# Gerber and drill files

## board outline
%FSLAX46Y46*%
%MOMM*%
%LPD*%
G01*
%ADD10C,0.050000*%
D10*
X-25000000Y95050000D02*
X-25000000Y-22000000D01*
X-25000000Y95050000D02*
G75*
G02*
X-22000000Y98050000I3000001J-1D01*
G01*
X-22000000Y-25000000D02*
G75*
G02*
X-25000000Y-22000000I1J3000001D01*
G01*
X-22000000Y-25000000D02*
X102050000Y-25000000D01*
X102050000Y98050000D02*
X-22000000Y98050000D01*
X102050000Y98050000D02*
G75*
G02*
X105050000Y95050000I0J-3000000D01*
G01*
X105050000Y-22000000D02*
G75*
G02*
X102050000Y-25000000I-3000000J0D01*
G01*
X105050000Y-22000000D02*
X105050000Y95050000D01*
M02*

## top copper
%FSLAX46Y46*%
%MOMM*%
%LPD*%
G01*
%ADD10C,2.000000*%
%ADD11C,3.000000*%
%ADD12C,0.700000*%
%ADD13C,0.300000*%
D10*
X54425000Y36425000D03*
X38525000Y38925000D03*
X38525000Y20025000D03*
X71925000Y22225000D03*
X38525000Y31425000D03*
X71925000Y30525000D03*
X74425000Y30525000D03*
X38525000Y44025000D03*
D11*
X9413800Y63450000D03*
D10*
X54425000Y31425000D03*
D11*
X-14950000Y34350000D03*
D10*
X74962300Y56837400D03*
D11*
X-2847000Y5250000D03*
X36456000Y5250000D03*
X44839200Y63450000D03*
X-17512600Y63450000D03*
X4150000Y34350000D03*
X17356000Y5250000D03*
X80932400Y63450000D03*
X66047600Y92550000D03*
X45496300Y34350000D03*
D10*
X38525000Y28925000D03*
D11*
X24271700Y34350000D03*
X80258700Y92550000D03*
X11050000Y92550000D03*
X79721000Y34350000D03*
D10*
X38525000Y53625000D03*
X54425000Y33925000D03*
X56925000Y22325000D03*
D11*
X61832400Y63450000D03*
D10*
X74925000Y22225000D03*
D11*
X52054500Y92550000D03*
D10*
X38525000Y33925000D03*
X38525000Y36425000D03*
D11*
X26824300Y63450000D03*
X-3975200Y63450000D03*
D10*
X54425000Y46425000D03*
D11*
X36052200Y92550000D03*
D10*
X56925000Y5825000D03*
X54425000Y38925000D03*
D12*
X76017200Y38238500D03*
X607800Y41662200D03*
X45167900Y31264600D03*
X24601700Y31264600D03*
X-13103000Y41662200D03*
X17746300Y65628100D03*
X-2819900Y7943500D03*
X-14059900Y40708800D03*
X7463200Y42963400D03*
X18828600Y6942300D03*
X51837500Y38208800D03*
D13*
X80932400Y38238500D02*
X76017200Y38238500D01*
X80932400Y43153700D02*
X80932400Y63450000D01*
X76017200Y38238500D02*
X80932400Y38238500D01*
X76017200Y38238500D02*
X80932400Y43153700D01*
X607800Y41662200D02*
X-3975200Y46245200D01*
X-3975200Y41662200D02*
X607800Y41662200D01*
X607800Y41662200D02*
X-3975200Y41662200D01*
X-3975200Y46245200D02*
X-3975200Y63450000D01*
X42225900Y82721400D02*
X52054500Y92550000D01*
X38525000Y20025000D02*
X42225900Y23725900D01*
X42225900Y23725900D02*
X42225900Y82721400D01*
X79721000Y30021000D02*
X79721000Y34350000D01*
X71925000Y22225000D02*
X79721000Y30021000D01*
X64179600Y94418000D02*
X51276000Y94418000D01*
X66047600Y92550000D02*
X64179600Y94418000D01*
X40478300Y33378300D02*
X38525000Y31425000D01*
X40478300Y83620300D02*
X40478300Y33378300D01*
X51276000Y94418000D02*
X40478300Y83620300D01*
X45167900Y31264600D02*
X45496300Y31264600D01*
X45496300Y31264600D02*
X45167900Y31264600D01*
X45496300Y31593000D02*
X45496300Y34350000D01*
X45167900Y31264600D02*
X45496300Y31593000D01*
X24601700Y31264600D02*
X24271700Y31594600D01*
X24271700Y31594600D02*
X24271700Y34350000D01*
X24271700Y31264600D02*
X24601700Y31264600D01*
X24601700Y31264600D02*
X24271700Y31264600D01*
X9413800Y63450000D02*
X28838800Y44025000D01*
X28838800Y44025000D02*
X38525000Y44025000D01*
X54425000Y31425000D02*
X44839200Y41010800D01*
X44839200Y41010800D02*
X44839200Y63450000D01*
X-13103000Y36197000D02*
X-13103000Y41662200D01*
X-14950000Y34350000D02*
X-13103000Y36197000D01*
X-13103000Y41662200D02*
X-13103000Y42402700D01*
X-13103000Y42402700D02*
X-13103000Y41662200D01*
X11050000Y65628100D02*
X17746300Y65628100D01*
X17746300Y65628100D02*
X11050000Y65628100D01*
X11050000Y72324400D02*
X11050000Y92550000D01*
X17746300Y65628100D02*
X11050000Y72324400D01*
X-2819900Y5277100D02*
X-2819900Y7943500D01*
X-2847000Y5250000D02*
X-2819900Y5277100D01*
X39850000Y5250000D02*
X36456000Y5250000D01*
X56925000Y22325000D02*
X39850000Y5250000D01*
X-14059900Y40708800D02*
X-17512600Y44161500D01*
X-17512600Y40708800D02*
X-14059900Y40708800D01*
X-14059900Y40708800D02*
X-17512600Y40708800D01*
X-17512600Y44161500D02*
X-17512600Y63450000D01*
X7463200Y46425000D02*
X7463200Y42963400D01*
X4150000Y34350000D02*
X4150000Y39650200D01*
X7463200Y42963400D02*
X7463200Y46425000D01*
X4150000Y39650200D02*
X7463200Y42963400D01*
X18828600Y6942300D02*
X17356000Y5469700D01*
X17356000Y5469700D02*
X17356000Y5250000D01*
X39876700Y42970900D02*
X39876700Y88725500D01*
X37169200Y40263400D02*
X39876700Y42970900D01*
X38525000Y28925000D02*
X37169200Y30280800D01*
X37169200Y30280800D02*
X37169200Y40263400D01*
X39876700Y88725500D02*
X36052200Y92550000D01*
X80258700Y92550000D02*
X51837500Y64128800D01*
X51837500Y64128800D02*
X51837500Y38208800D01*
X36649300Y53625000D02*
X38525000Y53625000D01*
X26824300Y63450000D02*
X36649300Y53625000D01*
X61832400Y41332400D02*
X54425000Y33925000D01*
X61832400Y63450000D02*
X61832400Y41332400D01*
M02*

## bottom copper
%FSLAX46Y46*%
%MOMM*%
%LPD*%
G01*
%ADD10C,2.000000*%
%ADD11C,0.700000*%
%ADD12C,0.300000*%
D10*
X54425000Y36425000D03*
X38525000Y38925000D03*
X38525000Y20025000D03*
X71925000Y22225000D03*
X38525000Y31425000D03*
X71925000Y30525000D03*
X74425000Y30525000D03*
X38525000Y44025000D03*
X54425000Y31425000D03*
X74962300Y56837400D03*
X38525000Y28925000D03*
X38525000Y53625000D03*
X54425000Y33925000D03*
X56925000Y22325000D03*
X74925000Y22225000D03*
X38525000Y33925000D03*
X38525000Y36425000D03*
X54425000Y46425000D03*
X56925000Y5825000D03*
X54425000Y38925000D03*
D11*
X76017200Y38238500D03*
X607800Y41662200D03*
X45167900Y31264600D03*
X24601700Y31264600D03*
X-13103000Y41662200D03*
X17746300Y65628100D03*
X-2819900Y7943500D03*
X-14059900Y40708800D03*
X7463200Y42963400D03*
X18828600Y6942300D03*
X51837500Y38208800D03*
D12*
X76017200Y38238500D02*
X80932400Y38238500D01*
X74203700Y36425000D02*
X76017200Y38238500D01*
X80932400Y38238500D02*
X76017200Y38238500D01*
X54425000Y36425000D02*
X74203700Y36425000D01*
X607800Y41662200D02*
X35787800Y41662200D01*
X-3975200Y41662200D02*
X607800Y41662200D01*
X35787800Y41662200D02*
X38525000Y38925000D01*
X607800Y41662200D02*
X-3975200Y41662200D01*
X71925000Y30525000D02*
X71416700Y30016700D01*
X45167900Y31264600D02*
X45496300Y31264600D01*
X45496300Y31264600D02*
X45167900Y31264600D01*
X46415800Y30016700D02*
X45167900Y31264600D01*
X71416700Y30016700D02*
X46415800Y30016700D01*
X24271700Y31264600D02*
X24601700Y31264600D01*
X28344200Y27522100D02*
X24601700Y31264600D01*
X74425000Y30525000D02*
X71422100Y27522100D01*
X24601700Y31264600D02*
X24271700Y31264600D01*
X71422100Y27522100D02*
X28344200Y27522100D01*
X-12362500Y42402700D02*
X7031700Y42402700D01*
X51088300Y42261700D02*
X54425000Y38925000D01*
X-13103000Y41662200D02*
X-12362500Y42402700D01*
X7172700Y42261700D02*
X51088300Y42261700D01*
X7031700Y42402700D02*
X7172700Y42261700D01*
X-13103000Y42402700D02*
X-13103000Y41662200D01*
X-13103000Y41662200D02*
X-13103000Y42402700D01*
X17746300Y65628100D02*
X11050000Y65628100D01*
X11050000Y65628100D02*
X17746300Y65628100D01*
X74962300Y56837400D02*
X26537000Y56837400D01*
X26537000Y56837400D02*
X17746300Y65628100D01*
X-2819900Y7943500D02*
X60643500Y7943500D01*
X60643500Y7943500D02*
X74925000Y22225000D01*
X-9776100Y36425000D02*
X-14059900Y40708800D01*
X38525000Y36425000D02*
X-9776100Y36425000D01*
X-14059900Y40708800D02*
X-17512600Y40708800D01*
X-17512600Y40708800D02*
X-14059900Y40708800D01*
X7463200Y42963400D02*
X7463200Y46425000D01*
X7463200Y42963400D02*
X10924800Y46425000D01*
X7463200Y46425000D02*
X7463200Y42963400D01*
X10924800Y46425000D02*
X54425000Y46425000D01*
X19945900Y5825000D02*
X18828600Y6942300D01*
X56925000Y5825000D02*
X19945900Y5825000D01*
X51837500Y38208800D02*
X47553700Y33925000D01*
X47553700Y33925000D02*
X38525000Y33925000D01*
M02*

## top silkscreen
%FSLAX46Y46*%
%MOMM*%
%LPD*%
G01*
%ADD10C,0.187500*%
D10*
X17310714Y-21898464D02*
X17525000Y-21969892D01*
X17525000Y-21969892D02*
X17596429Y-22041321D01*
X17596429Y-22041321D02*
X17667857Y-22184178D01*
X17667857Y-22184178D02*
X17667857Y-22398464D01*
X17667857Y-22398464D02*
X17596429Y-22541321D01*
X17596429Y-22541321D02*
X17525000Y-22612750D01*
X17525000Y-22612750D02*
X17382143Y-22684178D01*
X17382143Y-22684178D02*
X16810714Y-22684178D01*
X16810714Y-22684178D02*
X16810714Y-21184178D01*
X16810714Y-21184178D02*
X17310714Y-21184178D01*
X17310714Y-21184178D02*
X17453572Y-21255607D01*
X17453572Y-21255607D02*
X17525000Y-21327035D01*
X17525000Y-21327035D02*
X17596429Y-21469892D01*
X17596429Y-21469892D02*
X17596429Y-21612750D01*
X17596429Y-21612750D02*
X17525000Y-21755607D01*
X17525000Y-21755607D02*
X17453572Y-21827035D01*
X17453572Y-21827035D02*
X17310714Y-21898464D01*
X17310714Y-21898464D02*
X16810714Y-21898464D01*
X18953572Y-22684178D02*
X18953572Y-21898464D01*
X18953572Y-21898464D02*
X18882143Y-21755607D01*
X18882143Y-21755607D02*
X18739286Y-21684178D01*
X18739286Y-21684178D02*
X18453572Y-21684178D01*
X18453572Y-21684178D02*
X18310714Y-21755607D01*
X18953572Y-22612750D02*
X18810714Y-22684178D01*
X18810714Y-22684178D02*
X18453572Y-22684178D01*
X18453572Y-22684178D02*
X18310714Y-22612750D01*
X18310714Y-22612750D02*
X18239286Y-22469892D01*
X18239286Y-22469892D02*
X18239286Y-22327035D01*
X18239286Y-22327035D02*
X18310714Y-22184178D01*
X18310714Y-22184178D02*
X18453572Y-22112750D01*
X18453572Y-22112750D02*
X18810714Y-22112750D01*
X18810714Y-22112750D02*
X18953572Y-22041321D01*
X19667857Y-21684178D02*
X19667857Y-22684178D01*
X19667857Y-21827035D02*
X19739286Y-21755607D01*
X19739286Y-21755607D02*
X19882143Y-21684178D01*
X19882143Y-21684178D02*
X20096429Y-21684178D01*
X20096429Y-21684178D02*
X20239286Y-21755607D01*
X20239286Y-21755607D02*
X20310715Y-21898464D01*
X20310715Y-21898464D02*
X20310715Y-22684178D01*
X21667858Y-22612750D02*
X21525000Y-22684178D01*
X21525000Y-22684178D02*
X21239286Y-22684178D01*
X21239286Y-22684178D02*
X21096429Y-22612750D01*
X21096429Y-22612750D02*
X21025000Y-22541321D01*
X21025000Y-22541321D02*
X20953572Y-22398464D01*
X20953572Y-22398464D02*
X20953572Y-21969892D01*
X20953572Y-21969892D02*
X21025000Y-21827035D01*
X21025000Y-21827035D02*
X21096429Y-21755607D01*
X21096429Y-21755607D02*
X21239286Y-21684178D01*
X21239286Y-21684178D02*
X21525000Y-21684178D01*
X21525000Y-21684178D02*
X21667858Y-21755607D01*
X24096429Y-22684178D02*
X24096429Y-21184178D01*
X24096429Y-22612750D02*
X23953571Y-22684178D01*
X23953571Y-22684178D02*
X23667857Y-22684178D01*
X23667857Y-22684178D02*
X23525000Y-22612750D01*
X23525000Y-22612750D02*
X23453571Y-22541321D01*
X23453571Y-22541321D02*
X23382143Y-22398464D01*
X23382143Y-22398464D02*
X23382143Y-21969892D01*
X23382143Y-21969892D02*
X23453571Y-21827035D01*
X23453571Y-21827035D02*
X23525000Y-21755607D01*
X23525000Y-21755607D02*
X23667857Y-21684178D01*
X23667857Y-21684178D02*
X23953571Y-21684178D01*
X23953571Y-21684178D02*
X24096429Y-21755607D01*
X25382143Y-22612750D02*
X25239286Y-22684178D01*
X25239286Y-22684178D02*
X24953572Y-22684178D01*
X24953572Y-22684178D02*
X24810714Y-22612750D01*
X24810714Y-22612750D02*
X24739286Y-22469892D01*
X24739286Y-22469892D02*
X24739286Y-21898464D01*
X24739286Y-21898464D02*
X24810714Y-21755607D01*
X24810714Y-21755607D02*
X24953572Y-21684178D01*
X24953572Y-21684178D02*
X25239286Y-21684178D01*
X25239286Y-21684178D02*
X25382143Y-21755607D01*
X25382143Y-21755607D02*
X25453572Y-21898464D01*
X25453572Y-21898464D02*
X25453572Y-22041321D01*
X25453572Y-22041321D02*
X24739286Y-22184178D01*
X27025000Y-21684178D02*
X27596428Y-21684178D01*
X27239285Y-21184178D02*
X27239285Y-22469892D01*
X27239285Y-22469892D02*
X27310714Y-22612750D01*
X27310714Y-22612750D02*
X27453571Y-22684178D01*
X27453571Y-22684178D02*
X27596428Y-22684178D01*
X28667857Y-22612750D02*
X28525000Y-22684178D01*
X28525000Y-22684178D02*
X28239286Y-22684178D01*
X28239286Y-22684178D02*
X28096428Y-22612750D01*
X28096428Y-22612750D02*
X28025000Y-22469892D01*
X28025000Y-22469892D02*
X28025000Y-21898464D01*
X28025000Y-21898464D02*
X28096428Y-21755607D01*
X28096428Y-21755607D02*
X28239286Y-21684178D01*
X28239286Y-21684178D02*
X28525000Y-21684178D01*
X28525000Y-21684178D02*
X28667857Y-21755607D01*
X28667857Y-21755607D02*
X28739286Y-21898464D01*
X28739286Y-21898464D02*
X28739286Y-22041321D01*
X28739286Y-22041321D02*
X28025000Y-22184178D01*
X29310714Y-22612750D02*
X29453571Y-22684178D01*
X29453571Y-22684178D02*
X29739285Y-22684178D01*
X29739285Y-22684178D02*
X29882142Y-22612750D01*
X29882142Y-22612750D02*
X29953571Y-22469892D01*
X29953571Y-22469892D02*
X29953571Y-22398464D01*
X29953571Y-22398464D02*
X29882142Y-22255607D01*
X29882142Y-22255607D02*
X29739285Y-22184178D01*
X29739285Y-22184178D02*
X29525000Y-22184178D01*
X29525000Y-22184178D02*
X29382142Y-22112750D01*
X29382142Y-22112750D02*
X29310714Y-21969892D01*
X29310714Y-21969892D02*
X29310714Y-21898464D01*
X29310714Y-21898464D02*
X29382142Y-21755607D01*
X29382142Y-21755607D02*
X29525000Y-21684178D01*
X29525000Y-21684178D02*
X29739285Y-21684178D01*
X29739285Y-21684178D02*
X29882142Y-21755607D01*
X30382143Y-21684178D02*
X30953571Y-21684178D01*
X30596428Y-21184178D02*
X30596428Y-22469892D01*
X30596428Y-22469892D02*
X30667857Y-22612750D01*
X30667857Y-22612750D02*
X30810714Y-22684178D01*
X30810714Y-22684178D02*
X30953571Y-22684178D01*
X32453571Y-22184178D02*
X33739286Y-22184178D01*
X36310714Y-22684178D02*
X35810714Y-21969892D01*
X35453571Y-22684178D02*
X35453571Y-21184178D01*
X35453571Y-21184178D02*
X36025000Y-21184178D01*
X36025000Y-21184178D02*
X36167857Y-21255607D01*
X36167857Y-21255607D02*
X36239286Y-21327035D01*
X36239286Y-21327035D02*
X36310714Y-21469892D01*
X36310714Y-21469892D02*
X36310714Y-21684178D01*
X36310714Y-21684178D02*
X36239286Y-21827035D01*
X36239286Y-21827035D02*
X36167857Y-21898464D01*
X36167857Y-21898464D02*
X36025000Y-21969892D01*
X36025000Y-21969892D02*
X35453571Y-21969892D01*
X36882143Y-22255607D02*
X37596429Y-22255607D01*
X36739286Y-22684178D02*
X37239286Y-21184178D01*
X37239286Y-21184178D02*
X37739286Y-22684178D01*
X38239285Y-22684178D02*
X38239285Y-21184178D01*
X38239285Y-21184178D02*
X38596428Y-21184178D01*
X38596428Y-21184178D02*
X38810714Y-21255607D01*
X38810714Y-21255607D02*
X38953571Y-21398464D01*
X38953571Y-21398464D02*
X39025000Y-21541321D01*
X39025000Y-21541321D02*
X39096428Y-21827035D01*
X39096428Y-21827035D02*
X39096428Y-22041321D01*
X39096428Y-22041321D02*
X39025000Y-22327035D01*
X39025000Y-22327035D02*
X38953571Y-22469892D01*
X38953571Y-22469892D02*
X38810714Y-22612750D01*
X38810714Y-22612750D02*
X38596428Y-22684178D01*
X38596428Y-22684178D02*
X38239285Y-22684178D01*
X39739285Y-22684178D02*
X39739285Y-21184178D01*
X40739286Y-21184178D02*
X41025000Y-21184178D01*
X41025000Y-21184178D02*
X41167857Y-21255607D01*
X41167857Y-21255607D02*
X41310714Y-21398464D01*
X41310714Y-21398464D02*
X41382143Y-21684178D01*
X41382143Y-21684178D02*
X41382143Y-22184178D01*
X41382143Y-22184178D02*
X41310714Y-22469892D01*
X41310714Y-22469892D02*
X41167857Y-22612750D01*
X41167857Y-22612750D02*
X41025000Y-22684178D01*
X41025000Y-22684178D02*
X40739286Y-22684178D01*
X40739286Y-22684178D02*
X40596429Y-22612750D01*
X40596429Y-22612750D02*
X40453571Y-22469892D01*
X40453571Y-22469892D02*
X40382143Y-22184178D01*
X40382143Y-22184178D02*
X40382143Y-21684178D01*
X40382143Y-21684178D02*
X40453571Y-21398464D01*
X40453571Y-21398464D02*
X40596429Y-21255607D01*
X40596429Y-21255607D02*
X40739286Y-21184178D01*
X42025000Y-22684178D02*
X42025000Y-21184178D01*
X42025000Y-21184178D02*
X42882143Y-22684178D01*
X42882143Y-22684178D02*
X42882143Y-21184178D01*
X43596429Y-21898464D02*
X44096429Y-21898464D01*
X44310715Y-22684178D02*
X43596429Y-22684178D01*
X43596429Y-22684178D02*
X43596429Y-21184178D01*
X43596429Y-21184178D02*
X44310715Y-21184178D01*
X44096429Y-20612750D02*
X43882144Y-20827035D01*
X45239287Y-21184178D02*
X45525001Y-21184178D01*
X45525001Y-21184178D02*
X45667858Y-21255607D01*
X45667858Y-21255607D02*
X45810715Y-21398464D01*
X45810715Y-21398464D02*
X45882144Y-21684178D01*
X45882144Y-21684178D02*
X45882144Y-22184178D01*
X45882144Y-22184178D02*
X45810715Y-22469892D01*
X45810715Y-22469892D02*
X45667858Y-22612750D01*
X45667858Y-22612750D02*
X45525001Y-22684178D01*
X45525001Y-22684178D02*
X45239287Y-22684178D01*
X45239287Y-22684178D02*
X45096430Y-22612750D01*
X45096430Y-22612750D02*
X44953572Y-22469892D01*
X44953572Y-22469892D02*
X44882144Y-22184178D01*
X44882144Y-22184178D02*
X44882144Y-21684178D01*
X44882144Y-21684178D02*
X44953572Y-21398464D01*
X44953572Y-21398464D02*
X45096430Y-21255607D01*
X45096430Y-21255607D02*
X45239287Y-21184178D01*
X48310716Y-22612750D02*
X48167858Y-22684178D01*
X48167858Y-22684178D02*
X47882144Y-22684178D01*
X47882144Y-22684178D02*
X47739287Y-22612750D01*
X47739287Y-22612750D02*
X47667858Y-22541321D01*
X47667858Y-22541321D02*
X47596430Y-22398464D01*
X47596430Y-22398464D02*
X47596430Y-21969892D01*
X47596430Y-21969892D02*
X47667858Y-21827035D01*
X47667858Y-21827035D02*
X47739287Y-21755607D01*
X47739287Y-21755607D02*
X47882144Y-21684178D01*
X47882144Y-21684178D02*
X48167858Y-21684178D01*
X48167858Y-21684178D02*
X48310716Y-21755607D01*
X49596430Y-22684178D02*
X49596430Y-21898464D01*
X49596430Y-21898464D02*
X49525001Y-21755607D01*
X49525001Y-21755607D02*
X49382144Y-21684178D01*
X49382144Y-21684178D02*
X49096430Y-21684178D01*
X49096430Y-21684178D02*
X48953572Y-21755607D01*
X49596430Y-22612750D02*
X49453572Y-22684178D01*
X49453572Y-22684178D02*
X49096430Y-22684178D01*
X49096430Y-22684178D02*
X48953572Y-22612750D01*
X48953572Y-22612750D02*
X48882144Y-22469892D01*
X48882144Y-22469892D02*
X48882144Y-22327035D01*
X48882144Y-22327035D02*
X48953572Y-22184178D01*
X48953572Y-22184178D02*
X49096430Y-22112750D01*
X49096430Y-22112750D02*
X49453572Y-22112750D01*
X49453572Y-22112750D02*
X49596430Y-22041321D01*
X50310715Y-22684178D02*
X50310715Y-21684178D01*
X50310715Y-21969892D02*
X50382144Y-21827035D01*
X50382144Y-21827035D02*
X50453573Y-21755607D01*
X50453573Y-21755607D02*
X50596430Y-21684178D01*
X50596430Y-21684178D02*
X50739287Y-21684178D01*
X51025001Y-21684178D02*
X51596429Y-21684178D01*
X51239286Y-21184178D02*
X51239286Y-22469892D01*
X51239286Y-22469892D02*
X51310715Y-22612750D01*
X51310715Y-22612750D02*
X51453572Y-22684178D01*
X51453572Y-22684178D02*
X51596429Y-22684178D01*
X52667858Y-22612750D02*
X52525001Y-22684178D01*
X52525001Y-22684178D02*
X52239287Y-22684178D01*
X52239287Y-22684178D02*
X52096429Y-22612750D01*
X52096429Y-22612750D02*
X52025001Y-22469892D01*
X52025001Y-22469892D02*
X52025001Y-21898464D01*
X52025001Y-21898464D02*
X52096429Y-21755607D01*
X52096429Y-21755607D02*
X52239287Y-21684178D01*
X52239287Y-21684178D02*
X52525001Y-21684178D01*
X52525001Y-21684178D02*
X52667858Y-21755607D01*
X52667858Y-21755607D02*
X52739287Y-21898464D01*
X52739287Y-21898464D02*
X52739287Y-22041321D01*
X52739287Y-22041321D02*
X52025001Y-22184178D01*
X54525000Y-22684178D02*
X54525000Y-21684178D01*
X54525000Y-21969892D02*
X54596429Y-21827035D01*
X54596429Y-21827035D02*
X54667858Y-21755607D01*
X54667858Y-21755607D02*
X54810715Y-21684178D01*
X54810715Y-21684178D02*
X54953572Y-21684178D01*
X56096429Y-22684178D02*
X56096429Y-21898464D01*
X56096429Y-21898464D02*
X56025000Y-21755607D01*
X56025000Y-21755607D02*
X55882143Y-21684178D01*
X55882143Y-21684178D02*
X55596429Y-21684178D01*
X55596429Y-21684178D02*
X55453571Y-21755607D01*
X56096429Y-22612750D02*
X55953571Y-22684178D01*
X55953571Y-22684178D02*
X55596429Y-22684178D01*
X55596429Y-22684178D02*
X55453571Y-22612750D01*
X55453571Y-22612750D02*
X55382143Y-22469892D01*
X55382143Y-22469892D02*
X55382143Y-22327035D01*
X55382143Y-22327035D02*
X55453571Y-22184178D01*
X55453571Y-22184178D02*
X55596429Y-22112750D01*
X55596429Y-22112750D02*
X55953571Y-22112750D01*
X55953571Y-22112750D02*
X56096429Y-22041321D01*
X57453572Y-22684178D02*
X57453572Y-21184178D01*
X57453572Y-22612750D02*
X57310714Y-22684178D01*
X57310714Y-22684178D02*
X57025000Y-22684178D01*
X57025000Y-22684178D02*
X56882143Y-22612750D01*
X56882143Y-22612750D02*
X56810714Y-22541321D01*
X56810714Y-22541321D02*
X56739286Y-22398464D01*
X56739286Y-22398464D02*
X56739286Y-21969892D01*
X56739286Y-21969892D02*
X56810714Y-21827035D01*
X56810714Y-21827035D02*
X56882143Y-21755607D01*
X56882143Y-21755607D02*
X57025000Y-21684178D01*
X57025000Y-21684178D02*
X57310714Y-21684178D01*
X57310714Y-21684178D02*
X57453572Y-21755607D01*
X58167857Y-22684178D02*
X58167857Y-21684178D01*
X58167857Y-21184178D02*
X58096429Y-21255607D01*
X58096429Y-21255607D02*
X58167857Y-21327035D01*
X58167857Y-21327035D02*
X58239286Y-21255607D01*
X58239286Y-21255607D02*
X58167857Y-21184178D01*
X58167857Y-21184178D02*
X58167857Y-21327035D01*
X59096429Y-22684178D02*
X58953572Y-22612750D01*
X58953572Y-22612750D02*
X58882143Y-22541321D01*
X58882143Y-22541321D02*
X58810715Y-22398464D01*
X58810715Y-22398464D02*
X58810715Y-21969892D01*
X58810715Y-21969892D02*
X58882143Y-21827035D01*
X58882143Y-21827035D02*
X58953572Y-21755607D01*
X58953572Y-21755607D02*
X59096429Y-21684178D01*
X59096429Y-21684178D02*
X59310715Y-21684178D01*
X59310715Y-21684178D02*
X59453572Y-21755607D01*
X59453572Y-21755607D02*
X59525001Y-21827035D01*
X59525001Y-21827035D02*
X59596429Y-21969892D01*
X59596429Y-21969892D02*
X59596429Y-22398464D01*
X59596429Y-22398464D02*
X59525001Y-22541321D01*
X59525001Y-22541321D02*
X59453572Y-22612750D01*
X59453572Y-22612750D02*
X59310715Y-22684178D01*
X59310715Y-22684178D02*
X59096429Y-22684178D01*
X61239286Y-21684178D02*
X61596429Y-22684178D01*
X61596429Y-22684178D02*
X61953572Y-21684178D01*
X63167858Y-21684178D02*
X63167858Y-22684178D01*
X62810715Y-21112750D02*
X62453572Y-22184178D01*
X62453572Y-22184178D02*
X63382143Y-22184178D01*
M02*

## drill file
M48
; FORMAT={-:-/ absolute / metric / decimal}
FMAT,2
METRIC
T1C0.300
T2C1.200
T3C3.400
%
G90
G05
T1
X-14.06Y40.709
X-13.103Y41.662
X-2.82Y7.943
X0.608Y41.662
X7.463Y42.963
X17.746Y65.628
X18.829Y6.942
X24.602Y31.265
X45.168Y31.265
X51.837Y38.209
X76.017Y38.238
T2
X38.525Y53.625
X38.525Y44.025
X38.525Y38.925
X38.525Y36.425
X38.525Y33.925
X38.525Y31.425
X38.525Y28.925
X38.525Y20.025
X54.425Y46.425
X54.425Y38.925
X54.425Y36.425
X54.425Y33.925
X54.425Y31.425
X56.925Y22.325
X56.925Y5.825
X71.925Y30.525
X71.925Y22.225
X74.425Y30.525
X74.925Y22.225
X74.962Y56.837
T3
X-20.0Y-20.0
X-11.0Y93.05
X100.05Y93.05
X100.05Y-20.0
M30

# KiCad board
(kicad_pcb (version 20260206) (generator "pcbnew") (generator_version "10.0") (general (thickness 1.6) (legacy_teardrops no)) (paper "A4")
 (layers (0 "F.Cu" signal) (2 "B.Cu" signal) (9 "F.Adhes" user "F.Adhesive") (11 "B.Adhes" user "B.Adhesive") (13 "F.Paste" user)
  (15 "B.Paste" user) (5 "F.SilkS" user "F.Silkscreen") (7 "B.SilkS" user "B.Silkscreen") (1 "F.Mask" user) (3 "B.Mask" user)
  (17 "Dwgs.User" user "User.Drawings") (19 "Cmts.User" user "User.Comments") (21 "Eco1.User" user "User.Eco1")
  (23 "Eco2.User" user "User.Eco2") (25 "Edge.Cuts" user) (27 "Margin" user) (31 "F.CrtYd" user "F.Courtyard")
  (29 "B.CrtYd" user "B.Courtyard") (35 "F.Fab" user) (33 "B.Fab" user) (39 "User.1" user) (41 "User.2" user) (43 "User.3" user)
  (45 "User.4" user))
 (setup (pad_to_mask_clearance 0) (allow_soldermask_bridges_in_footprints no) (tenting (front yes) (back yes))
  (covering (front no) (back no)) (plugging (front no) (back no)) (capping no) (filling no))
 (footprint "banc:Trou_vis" (layer "F.Cu") (at 100.05 -93.05)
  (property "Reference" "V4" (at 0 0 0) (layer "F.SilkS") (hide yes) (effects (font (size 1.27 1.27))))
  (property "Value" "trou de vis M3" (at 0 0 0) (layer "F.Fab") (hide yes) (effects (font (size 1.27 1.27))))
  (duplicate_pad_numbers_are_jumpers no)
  (pad "" np_thru_hole circle (at 0 0) (size 3.4 3.4) (drill 3.4) (layers "*.Cu" "*.Mask")))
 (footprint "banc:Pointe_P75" (layer "F.Cu") (at 54.425 -36.425)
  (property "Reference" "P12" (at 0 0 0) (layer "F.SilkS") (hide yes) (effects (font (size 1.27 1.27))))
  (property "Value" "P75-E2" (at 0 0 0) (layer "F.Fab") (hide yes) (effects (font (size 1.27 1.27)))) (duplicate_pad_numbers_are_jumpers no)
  (pad "1" thru_hole circle (at 0 0) (size 2 2) (drill 1.2) (layers "*.Cu" "*.Mask") (remove_unused_layers no) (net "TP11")))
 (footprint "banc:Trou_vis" (layer "F.Cu") (at 100.05 20)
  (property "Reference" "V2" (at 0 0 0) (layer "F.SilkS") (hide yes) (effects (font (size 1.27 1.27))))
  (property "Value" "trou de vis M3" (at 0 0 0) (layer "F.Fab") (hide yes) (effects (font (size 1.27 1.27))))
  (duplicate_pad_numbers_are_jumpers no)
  (pad "" np_thru_hole circle (at 0 0) (size 3.4 3.4) (drill 3.4) (layers "*.Cu" "*.Mask")))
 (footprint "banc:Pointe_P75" (layer "F.Cu") (at 38.525 -38.925)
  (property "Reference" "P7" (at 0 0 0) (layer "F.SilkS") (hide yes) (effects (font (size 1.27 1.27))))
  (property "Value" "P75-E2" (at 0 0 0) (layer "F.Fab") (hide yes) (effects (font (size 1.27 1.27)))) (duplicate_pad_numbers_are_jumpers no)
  (pad "1" thru_hole circle (at 0 0) (size 2 2) (drill 1.2) (layers "*.Cu" "*.Mask") (remove_unused_layers no) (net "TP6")))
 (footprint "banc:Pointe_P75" (layer "F.Cu") (at 38.525 -20.025)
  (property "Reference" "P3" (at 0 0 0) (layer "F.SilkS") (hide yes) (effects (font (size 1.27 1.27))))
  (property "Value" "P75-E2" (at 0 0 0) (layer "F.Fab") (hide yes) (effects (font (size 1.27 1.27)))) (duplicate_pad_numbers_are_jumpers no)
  (pad "1" thru_hole circle (at 0 0) (size 2 2) (drill 1.2) (layers "*.Cu" "*.Mask") (remove_unused_layers no) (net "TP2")))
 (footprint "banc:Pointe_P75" (layer "F.Cu") (at 71.925 -22.225)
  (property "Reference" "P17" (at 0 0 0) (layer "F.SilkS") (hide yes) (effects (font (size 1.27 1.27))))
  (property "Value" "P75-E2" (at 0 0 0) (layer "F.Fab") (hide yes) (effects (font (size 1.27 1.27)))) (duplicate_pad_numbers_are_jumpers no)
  (pad "1" thru_hole circle (at 0 0) (size 2 2) (drill 1.2) (layers "*.Cu" "*.Mask") (remove_unused_layers no) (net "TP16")))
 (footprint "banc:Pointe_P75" (layer "F.Cu") (at 38.525 -31.425)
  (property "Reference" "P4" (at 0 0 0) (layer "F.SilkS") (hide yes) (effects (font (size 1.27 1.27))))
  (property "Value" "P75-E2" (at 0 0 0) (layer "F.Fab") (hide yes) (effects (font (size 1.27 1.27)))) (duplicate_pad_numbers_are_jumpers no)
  (pad "1" thru_hole circle (at 0 0) (size 2 2) (drill 1.2) (layers "*.Cu" "*.Mask") (remove_unused_layers no) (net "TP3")))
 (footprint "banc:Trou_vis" (layer "F.Cu") (at -20 20)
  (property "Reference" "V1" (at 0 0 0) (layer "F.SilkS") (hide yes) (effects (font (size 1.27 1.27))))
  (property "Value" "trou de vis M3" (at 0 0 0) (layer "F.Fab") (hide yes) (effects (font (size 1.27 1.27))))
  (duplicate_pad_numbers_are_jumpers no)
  (pad "" np_thru_hole circle (at 0 0) (size 3.4 3.4) (drill 3.4) (layers "*.Cu" "*.Mask")))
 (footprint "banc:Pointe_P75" (layer "F.Cu") (at 71.925 -30.525)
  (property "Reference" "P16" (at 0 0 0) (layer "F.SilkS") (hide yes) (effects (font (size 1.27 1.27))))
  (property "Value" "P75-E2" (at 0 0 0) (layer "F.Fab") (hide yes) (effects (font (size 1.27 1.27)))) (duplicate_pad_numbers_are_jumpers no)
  (pad "1" thru_hole circle (at 0 0) (size 2 2) (drill 1.2) (layers "*.Cu" "*.Mask") (remove_unused_layers no) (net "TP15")))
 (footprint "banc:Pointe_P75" (layer "F.Cu") (at 74.425 -30.525)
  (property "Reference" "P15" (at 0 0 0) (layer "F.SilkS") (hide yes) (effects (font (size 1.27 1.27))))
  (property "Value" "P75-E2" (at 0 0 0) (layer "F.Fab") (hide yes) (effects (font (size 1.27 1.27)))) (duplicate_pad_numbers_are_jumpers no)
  (pad "1" thru_hole circle (at 0 0) (size 2 2) (drill 1.2) (layers "*.Cu" "*.Mask") (remove_unused_layers no) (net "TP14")))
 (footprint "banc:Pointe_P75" (layer "F.Cu") (at 38.525 -44.025)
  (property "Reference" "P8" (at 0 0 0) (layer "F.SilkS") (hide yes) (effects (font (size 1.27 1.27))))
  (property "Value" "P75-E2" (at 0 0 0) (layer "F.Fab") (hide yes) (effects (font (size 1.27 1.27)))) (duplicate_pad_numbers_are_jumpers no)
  (pad "1" thru_hole circle (at 0 0) (size 2 2) (drill 1.2) (layers "*.Cu" "*.Mask") (remove_unused_layers no) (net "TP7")))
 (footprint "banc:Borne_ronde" (layer "F.Cu") (at 9.4138 -63.45)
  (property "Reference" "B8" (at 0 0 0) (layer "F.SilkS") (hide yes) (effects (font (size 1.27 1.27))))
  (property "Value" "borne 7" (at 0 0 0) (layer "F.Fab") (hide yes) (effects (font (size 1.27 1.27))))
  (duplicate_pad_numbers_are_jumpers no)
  (pad "1" smd circle (at 0 0) (size 3 3) (layers "F.Cu" "F.Mask") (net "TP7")))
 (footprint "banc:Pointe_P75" (layer "F.Cu") (at 54.425 -31.425)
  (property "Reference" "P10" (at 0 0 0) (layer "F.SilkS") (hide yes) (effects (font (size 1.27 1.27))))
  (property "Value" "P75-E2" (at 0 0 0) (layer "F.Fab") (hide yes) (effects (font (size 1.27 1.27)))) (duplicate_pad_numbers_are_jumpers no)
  (pad "1" thru_hole circle (at 0 0) (size 2 2) (drill 1.2) (layers "*.Cu" "*.Mask") (remove_unused_layers no) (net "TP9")))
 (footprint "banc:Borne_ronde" (layer "F.Cu") (at -14.95 -34.35)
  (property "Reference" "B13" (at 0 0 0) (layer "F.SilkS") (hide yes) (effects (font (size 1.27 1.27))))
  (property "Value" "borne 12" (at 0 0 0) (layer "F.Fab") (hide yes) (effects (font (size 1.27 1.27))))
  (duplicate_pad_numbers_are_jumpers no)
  (pad "1" smd circle (at 0 0) (size 3 3) (layers "F.Cu" "F.Mask") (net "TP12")))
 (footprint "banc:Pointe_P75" (layer "F.Cu") (at 74.9623 -56.8374)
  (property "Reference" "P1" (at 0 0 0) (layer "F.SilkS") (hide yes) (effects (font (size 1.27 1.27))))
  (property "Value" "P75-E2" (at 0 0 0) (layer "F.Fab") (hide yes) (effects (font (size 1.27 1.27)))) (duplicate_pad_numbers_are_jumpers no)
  (pad "1" thru_hole circle (at 0 0) (size 2 2) (drill 1.2) (layers "*.Cu" "*.Mask") (remove_unused_layers no) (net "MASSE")))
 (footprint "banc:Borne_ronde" (layer "F.Cu") (at -2.847 -5.25)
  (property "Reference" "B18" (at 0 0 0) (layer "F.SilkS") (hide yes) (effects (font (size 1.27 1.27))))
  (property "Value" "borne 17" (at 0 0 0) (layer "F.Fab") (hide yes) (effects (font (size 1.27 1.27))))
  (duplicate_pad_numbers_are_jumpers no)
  (pad "1" smd circle (at 0 0) (size 3 3) (layers "F.Cu" "F.Mask") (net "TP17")))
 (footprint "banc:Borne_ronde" (layer "F.Cu") (at 36.456 -5.25)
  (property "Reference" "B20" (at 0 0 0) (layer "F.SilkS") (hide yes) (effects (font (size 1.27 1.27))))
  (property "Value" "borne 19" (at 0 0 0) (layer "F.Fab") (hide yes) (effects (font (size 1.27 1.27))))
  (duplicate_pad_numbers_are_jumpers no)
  (pad "1" smd circle (at 0 0) (size 3 3) (layers "F.Cu" "F.Mask") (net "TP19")))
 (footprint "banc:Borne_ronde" (layer "F.Cu") (at 44.8392 -63.45)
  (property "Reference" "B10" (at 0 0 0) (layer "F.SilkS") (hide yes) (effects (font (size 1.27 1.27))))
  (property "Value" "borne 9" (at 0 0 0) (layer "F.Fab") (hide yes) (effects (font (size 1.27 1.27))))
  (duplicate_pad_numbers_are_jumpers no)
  (pad "1" smd circle (at 0 0) (size 3 3) (layers "F.Cu" "F.Mask") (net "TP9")))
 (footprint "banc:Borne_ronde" (layer "F.Cu") (at -17.5126 -63.45)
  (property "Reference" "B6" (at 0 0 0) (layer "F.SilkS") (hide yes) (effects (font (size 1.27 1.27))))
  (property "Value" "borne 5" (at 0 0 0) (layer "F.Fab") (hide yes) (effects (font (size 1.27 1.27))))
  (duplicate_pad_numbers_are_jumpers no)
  (pad "1" smd circle (at 0 0) (size 3 3) (layers "F.Cu" "F.Mask") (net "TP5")))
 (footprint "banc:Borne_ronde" (layer "F.Cu") (at 4.15 -34.35)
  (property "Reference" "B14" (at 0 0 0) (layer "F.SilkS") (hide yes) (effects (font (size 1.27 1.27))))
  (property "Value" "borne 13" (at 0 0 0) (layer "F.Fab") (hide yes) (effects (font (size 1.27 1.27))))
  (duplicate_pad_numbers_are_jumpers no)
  (pad "1" smd circle (at 0 0) (size 3 3) (layers "F.Cu" "F.Mask") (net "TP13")))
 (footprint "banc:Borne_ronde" (layer "F.Cu") (at 17.356 -5.25)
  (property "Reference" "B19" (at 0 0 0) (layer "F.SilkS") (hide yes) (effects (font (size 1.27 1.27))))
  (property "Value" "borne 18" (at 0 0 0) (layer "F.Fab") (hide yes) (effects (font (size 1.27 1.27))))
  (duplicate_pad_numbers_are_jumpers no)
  (pad "1" smd circle (at 0 0) (size 3 3) (layers "F.Cu" "F.Mask") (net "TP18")))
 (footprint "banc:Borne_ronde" (layer "F.Cu") (at 80.9324 -63.45)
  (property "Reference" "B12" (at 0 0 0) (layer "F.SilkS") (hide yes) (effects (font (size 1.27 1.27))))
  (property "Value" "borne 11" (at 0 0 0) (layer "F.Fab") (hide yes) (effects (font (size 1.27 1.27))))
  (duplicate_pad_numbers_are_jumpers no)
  (pad "1" smd circle (at 0 0) (size 3 3) (layers "F.Cu" "F.Mask") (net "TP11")))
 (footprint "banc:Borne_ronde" (layer "F.Cu") (at 66.0476 -92.55)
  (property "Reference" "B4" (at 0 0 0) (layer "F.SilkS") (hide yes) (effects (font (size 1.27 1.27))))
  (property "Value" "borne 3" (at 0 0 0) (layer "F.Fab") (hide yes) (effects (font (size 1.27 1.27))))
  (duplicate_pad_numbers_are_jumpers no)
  (pad "1" smd circle (at 0 0) (size 3 3) (layers "F.Cu" "F.Mask") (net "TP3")))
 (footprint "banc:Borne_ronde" (layer "F.Cu") (at 45.4963 -34.35)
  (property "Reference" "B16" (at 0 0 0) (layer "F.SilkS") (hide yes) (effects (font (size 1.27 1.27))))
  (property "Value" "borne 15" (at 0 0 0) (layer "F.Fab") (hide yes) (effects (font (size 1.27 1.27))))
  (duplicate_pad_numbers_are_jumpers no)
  (pad "1" smd circle (at 0 0) (size 3 3) (layers "F.Cu" "F.Mask") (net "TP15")))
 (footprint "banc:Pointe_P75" (layer "F.Cu") (at 38.525 -28.925)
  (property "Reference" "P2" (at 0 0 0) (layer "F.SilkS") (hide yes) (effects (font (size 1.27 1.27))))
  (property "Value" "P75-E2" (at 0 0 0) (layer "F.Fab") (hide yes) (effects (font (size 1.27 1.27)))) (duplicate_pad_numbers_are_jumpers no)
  (pad "1" thru_hole circle (at 0 0) (size 2 2) (drill 1.2) (layers "*.Cu" "*.Mask") (remove_unused_layers no) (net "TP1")))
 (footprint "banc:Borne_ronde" (layer "F.Cu") (at 24.2717 -34.35)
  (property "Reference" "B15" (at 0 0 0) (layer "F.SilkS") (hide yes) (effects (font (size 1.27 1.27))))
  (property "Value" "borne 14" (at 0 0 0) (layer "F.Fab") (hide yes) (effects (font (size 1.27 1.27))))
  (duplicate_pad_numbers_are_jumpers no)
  (pad "1" smd circle (at 0 0) (size 3 3) (layers "F.Cu" "F.Mask") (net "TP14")))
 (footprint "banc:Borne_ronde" (layer "F.Cu") (at 80.2587 -92.55)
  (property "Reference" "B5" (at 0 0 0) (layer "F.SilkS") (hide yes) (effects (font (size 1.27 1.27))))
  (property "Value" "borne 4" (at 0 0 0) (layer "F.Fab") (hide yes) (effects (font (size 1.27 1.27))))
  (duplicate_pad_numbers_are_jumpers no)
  (pad "1" smd circle (at 0 0) (size 3 3) (layers "F.Cu" "F.Mask") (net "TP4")))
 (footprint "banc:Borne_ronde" (layer "F.Cu") (at 11.05 -92.55)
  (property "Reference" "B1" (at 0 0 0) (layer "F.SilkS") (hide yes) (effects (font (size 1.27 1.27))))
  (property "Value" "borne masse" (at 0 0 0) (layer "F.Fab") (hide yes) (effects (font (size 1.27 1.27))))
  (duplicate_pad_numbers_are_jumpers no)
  (pad "1" smd circle (at 0 0) (size 3 3) (layers "F.Cu" "F.Mask") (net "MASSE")))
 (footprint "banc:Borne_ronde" (layer "F.Cu") (at 79.721 -34.35)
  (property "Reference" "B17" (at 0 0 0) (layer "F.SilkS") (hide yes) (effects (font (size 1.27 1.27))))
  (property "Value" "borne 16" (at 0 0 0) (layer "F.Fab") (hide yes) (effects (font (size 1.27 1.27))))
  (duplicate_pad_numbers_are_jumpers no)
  (pad "1" smd circle (at 0 0) (size 3 3) (layers "F.Cu" "F.Mask") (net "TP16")))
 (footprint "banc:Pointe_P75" (layer "F.Cu") (at 38.525 -53.625)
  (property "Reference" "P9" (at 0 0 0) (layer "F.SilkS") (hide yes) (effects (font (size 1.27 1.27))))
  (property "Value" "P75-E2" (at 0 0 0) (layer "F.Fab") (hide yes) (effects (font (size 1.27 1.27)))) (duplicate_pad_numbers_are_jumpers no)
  (pad "1" thru_hole circle (at 0 0) (size 2 2) (drill 1.2) (layers "*.Cu" "*.Mask") (remove_unused_layers no) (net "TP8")))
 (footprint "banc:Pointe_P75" (layer "F.Cu") (at 54.425 -33.925)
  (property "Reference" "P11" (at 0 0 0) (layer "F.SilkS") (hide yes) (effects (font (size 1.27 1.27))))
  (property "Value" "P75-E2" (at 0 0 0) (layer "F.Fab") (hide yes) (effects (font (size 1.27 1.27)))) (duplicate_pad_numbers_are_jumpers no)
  (pad "1" thru_hole circle (at 0 0) (size 2 2) (drill 1.2) (layers "*.Cu" "*.Mask") (remove_unused_layers no) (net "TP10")))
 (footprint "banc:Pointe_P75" (layer "F.Cu") (at 56.925 -22.325)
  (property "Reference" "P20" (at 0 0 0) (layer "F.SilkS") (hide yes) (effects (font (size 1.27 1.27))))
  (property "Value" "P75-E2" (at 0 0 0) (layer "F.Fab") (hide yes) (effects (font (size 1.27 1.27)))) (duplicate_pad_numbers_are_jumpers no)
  (pad "1" thru_hole circle (at 0 0) (size 2 2) (drill 1.2) (layers "*.Cu" "*.Mask") (remove_unused_layers no) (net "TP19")))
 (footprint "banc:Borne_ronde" (layer "F.Cu") (at 61.8324 -63.45)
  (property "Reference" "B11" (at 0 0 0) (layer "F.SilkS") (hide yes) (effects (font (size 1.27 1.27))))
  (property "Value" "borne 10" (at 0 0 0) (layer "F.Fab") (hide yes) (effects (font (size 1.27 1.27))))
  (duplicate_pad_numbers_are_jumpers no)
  (pad "1" smd circle (at 0 0) (size 3 3) (layers "F.Cu" "F.Mask") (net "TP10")))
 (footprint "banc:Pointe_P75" (layer "F.Cu") (at 74.925 -22.225)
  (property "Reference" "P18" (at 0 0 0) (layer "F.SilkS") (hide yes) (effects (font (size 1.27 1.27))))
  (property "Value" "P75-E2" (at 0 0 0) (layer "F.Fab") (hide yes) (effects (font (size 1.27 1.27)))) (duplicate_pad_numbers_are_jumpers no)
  (pad "1" thru_hole circle (at 0 0) (size 2 2) (drill 1.2) (layers "*.Cu" "*.Mask") (remove_unused_layers no) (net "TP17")))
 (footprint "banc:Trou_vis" (layer "F.Cu") (at -11 -93.05)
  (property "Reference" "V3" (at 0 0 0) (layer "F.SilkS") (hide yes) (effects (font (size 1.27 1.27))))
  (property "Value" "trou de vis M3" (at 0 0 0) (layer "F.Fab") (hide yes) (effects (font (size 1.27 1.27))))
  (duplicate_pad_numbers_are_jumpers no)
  (pad "" np_thru_hole circle (at 0 0) (size 3.4 3.4) (drill 3.4) (layers "*.Cu" "*.Mask")))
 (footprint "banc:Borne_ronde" (layer "F.Cu") (at 52.0545 -92.55)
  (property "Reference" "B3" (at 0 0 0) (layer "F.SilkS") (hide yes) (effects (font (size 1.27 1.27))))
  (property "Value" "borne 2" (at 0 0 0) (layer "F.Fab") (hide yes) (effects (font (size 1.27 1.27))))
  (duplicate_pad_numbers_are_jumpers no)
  (pad "1" smd circle (at 0 0) (size 3 3) (layers "F.Cu" "F.Mask") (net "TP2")))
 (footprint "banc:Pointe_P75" (layer "F.Cu") (at 38.525 -33.925)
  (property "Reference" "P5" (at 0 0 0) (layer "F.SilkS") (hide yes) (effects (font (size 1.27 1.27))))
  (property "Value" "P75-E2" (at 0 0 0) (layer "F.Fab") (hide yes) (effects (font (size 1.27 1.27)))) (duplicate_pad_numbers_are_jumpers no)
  (pad "1" thru_hole circle (at 0 0) (size 2 2) (drill 1.2) (layers "*.Cu" "*.Mask") (remove_unused_layers no) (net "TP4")))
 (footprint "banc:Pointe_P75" (layer "F.Cu") (at 38.525 -36.425)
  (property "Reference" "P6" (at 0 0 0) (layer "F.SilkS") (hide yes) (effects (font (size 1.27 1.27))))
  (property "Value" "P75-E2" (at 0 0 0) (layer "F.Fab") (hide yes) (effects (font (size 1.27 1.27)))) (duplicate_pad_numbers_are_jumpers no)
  (pad "1" thru_hole circle (at 0 0) (size 2 2) (drill 1.2) (layers "*.Cu" "*.Mask") (remove_unused_layers no) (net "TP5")))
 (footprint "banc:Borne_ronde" (layer "F.Cu") (at 26.8243 -63.45)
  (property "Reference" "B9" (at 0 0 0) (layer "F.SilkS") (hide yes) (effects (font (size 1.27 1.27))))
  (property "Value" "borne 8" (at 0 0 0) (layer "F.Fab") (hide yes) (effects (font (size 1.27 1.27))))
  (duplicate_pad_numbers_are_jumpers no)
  (pad "1" smd circle (at 0 0) (size 3 3) (layers "F.Cu" "F.Mask") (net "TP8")))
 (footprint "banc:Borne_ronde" (layer "F.Cu") (at -3.9752 -63.45)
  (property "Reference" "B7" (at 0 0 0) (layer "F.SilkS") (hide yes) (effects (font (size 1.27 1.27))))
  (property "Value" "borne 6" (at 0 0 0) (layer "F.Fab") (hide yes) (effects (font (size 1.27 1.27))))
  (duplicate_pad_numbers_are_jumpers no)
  (pad "1" smd circle (at 0 0) (size 3 3) (layers "F.Cu" "F.Mask") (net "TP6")))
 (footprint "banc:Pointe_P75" (layer "F.Cu") (at 54.425 -46.425)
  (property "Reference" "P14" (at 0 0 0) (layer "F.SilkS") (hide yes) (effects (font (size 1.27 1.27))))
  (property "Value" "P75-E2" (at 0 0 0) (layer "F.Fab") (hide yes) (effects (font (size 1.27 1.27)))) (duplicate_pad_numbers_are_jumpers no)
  (pad "1" thru_hole circle (at 0 0) (size 2 2) (drill 1.2) (layers "*.Cu" "*.Mask") (remove_unused_layers no) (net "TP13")))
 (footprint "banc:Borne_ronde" (layer "F.Cu") (at 36.0522 -92.55)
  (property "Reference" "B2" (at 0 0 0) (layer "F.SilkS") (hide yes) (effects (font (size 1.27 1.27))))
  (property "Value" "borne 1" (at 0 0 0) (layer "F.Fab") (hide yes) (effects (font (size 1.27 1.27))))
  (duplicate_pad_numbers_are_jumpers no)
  (pad "1" smd circle (at 0 0) (size 3 3) (layers "F.Cu" "F.Mask") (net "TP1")))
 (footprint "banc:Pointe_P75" (layer "F.Cu") (at 56.925 -5.825)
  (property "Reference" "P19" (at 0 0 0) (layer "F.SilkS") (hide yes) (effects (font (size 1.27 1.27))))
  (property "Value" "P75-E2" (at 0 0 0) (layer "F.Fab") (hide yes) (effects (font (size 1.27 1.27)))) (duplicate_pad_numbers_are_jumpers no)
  (pad "1" thru_hole circle (at 0 0) (size 2 2) (drill 1.2) (layers "*.Cu" "*.Mask") (remove_unused_layers no) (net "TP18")))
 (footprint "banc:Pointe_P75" (layer "F.Cu") (at 54.425 -38.925)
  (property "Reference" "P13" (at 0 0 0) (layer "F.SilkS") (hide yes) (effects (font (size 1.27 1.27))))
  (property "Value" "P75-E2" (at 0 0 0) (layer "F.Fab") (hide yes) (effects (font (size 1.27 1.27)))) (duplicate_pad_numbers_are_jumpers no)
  (pad "1" thru_hole circle (at 0 0) (size 2 2) (drill 1.2) (layers "*.Cu" "*.Mask") (remove_unused_layers no) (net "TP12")))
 (gr_line (start -25 -95.05) (end -25 22) (stroke (width 0.05) (type default)) (layer "Edge.Cuts"))
 (gr_arc (start -25 -95.05) (mid -24.12132 -97.17132) (end -22 -98.05) (stroke (width 0.05) (type default)) (layer "Edge.Cuts"))
 (gr_arc (start -22 25) (mid -24.12132 24.12132) (end -25 22) (stroke (width 0.05) (type default)) (layer "Edge.Cuts"))
 (gr_line (start -22 25) (end 102.05 25) (stroke (width 0.05) (type default)) (layer "Edge.Cuts"))
 (gr_line (start 102.05 -98.05) (end -22 -98.05) (stroke (width 0.05) (type default)) (layer "Edge.Cuts"))
 (gr_arc (start 102.05 -98.05) (mid 104.17132 -97.17132) (end 105.05 -95.05) (stroke (width 0.05) (type default)) (layer "Edge.Cuts"))
 (gr_arc (start 105.05 22) (mid 104.17132 24.12132) (end 102.05 25) (stroke (width 0.05) (type default)) (layer "Edge.Cuts"))
 (gr_line (start 105.05 22) (end 105.05 -95.05) (stroke (width 0.05) (type default)) (layer "Edge.Cuts"))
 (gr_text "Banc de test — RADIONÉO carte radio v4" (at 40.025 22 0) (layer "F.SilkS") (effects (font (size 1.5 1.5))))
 (segment (start 80.9324 -38.2385) (end 76.0172 -38.2385) (width 0.3) (layer "F.Cu") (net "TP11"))
 (segment (start 80.9324 -43.1537) (end 80.9324 -63.45) (width 0.3) (layer "F.Cu") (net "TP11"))
 (segment (start 76.0172 -38.2385) (end 80.9324 -38.2385) (width 0.3) (layer "F.Cu") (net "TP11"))
 (segment (start 76.0172 -38.2385) (end 80.9324 -43.1537) (width 0.3) (layer "F.Cu") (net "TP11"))
 (via (at 76.0172 -38.2385) (size 0.7) (drill 0.3) (layers "F.Cu" "B.Cu") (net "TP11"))
 (segment (start 76.0172 -38.2385) (end 80.9324 -38.2385) (width 0.3) (layer "B.Cu") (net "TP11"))
 (segment (start 74.2037 -36.425) (end 76.0172 -38.2385) (width 0.3) (layer "B.Cu") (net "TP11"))
 (segment (start 80.9324 -38.2385) (end 76.0172 -38.2385) (width 0.3) (layer "B.Cu") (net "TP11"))
 (segment (start 54.425 -36.425) (end 74.2037 -36.425) (width 0.3) (layer "B.Cu") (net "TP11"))
 (segment (start 0.6078 -41.6622) (end -3.9752 -46.2452) (width 0.3) (layer "F.Cu") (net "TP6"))
 (segment (start -3.9752 -41.6622) (end 0.6078 -41.6622) (width 0.3) (layer "F.Cu") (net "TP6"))
 (segment (start 0.6078 -41.6622) (end -3.9752 -41.6622) (width 0.3) (layer "F.Cu") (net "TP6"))
 (segment (start -3.9752 -46.2452) (end -3.9752 -63.45) (width 0.3) (layer "F.Cu") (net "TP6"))
 (via (at 0.6078 -41.6622) (size 0.7) (drill 0.3) (layers "F.Cu" "B.Cu") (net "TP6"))
 (segment (start 0.6078 -41.6622) (end 35.7878 -41.6622) (width 0.3) (layer "B.Cu") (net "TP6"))
 (segment (start -3.9752 -41.6622) (end 0.6078 -41.6622) (width 0.3) (layer "B.Cu") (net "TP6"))
 (segment (start 35.7878 -41.6622) (end 38.525 -38.925) (width 0.3) (layer "B.Cu") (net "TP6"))
 (segment (start 0.6078 -41.6622) (end -3.9752 -41.6622) (width 0.3) (layer "B.Cu") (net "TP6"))
 (segment (start 42.2259 -82.7214) (end 52.0545 -92.55) (width 0.3) (layer "F.Cu") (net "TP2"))
 (segment (start 38.525 -20.025) (end 42.2259 -23.7259) (width 0.3) (layer "F.Cu") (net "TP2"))
 (segment (start 42.2259 -23.7259) (end 42.2259 -82.7214) (width 0.3) (layer "F.Cu") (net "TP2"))
 (segment (start 79.721 -30.021) (end 79.721 -34.35) (width 0.3) (layer "F.Cu") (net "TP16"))
 (segment (start 71.925 -22.225) (end 79.721 -30.021) (width 0.3) (layer "F.Cu") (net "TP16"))
 (segment (start 64.1796 -94.418) (end 51.276 -94.418) (width 0.3) (layer "F.Cu") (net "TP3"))
 (segment (start 66.0476 -92.55) (end 64.1796 -94.418) (width 0.3) (layer "F.Cu") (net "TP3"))
 (segment (start 40.4783 -33.3783) (end 38.525 -31.425) (width 0.3) (layer "F.Cu") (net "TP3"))
 (segment (start 40.4783 -83.6203) (end 40.4783 -33.3783) (width 0.3) (layer "F.Cu") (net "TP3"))
 (segment (start 51.276 -94.418) (end 40.4783 -83.6203) (width 0.3) (layer "F.Cu") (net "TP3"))
 (segment (start 45.1679 -31.2646) (end 45.4963 -31.2646) (width 0.3) (layer "F.Cu") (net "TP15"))
 (segment (start 45.4963 -31.2646) (end 45.1679 -31.2646) (width 0.3) (layer "F.Cu") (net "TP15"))
 (segment (start 45.4963 -31.593) (end 45.4963 -34.35) (width 0.3) (layer "F.Cu") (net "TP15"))
 (segment (start 45.1679 -31.2646) (end 45.4963 -31.593) (width 0.3) (layer "F.Cu") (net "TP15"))
 (via (at 45.1679 -31.2646) (size 0.7) (drill 0.3) (layers "F.Cu" "B.Cu") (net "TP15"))
 (segment (start 71.925 -30.525) (end 71.4167 -30.0167) (width 0.3) (layer "B.Cu") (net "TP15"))
 (segment (start 45.1679 -31.2646) (end 45.4963 -31.2646) (width 0.3) (layer "B.Cu") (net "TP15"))
 (segment (start 45.4963 -31.2646) (end 45.1679 -31.2646) (width 0.3) (layer "B.Cu") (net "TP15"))
 (segment (start 46.4158 -30.0167) (end 45.1679 -31.2646) (width 0.3) (layer "B.Cu") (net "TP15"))
 (segment (start 71.4167 -30.0167) (end 46.4158 -30.0167) (width 0.3) (layer "B.Cu") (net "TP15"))
 (segment (start 24.6017 -31.2646) (end 24.2717 -31.5946) (width 0.3) (layer "F.Cu") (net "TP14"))
 (segment (start 24.2717 -31.5946) (end 24.2717 -34.35) (width 0.3) (layer "F.Cu") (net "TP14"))
 (segment (start 24.2717 -31.2646) (end 24.6017 -31.2646) (width 0.3) (layer "F.Cu") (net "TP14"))
 (segment (start 24.6017 -31.2646) (end 24.2717 -31.2646) (width 0.3) (layer "F.Cu") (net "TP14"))
 (via (at 24.6017 -31.2646) (size 0.7) (drill 0.3) (layers "F.Cu" "B.Cu") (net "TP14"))
 (segment (start 24.2717 -31.2646) (end 24.6017 -31.2646) (width 0.3) (layer "B.Cu") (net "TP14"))
 (segment (start 28.3442 -27.5221) (end 24.6017 -31.2646) (width 0.3) (layer "B.Cu") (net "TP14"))
 (segment (start 74.425 -30.525) (end 71.4221 -27.5221) (width 0.3) (layer "B.Cu") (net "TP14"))
 (segment (start 24.6017 -31.2646) (end 24.2717 -31.2646) (width 0.3) (layer "B.Cu") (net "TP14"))
 (segment (start 71.4221 -27.5221) (end 28.3442 -27.5221) (width 0.3) (layer "B.Cu") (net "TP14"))
 (segment (start 9.4138 -63.45) (end 28.8388 -44.025) (width 0.3) (layer "F.Cu") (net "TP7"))
 (segment (start 28.8388 -44.025) (end 38.525 -44.025) (width 0.3) (layer "F.Cu") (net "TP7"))
 (segment (start 54.425 -31.425) (end 44.8392 -41.0108) (width 0.3) (layer "F.Cu") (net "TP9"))
 (segment (start 44.8392 -41.0108) (end 44.8392 -63.45) (width 0.3) (layer "F.Cu") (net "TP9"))
 (segment (start -13.103 -36.197) (end -13.103 -41.6622) (width 0.3) (layer "F.Cu") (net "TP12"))
 (segment (start -14.95 -34.35) (end -13.103 -36.197) (width 0.3) (layer "F.Cu") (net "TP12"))
 (segment (start -13.103 -41.6622) (end -13.103 -42.4027) (width 0.3) (layer "F.Cu") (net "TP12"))
 (segment (start -13.103 -42.4027) (end -13.103 -41.6622) (width 0.3) (layer "F.Cu") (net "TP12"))
 (via (at -13.103 -41.6622) (size 0.7) (drill 0.3) (layers "F.Cu" "B.Cu") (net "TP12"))
 (segment (start -12.3625 -42.4027) (end 7.0317 -42.4027) (width 0.3) (layer "B.Cu") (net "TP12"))
 (segment (start 51.0883 -42.2617) (end 54.425 -38.925) (width 0.3) (layer "B.Cu") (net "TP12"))
 (segment (start -13.103 -41.6622) (end -12.3625 -42.4027) (width 0.3) (layer "B.Cu") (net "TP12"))
 (segment (start 7.1727 -42.2617) (end 51.0883 -42.2617) (width 0.3) (layer "B.Cu") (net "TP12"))
 (segment (start 7.0317 -42.4027) (end 7.1727 -42.2617) (width 0.3) (layer "B.Cu") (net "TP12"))
 (segment (start -13.103 -42.4027) (end -13.103 -41.6622) (width 0.3) (layer "B.Cu") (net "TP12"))
 (segment (start -13.103 -41.6622) (end -13.103 -42.4027) (width 0.3) (layer "B.Cu") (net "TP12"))
 (segment (start 11.05 -65.6281) (end 17.7463 -65.6281) (width 0.3) (layer "F.Cu") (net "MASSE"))
 (segment (start 17.7463 -65.6281) (end 11.05 -65.6281) (width 0.3) (layer "F.Cu") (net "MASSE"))
 (segment (start 11.05 -72.3244) (end 11.05 -92.55) (width 0.3) (layer "F.Cu") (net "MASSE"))
 (segment (start 17.7463 -65.6281) (end 11.05 -72.3244) (width 0.3) (layer "F.Cu") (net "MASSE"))
 (via (at 17.7463 -65.6281) (size 0.7) (drill 0.3) (layers "F.Cu" "B.Cu") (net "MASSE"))
 (segment (start 17.7463 -65.6281) (end 11.05 -65.6281) (width 0.3) (layer "B.Cu") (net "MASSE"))
 (segment (start 11.05 -65.6281) (end 17.7463 -65.6281) (width 0.3) (layer "B.Cu") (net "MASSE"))
 (segment (start 74.9623 -56.8374) (end 26.537 -56.8374) (width 0.3) (layer "B.Cu") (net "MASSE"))
 (segment (start 26.537 -56.8374) (end 17.7463 -65.6281) (width 0.3) (layer "B.Cu") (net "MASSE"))
 (segment (start -2.8199 -5.2771) (end -2.8199 -7.9435) (width 0.3) (layer "F.Cu") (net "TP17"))
 (segment (start -2.847 -5.25) (end -2.8199 -5.2771) (width 0.3) (layer "F.Cu") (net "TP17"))
 (via (at -2.8199 -7.9435) (size 0.7) (drill 0.3) (layers "F.Cu" "B.Cu") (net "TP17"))
 (segment (start -2.8199 -7.9435) (end 60.6435 -7.9435) (width 0.3) (layer "B.Cu") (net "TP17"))
 (segment (start 60.6435 -7.9435) (end 74.925 -22.225) (width 0.3) (layer "B.Cu") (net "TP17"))
 (segment (start 39.85 -5.25) (end 36.456 -5.25) (width 0.3) (layer "F.Cu") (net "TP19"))
 (segment (start 56.925 -22.325) (end 39.85 -5.25) (width 0.3) (layer "F.Cu") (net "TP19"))
 (segment (start -14.0599 -40.7088) (end -17.5126 -44.1615) (width 0.3) (layer "F.Cu") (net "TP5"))
 (segment (start -17.5126 -40.7088) (end -14.0599 -40.7088) (width 0.3) (layer "F.Cu") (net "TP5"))
 (segment (start -14.0599 -40.7088) (end -17.5126 -40.7088) (width 0.3) (layer "F.Cu") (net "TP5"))
 (segment (start -17.5126 -44.1615) (end -17.5126 -63.45) (width 0.3) (layer "F.Cu") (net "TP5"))
 (via (at -14.0599 -40.7088) (size 0.7) (drill 0.3) (layers "F.Cu" "B.Cu") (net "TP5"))
 (segment (start -9.7761 -36.425) (end -14.0599 -40.7088) (width 0.3) (layer "B.Cu") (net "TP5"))
 (segment (start 38.525 -36.425) (end -9.7761 -36.425) (width 0.3) (layer "B.Cu") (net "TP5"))
 (segment (start -14.0599 -40.7088) (end -17.5126 -40.7088) (width 0.3) (layer "B.Cu") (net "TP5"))
 (segment (start -17.5126 -40.7088) (end -14.0599 -40.7088) (width 0.3) (layer "B.Cu") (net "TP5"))
 (segment (start 7.4632 -46.425) (end 7.4632 -42.9634) (width 0.3) (layer "F.Cu") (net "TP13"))
 (segment (start 4.15 -34.35) (end 4.15 -39.6502) (width 0.3) (layer "F.Cu") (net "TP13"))
 (segment (start 7.4632 -42.9634) (end 7.4632 -46.425) (width 0.3) (layer "F.Cu") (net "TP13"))
 (segment (start 4.15 -39.6502) (end 7.4632 -42.9634) (width 0.3) (layer "F.Cu") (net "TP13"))
 (via (at 7.4632 -42.9634) (size 0.7) (drill 0.3) (layers "F.Cu" "B.Cu") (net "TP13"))
 (segment (start 7.4632 -42.9634) (end 7.4632 -46.425) (width 0.3) (layer "B.Cu") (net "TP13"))
 (segment (start 7.4632 -42.9634) (end 10.9248 -46.425) (width 0.3) (layer "B.Cu") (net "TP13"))
 (segment (start 7.4632 -46.425) (end 7.4632 -42.9634) (width 0.3) (layer "B.Cu") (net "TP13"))
 (segment (start 10.9248 -46.425) (end 54.425 -46.425) (width 0.3) (layer "B.Cu") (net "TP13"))
 (segment (start 18.8286 -6.9423) (end 17.356 -5.4697) (width 0.3) (layer "F.Cu") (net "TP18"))
 (segment (start 17.356 -5.4697) (end 17.356 -5.25) (width 0.3) (layer "F.Cu") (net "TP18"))
 (via (at 18.8286 -6.9423) (size 0.7) (drill 0.3) (layers "F.Cu" "B.Cu") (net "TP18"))
 (segment (start 19.9459 -5.825) (end 18.8286 -6.9423) (width 0.3) (layer "B.Cu") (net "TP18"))
 (segment (start 56.925 -5.825) (end 19.9459 -5.825) (width 0.3) (layer "B.Cu") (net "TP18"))
 (segment (start 39.8767 -42.9709) (end 39.8767 -88.7255) (width 0.3) (layer "F.Cu") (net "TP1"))
 (segment (start 37.1692 -40.2634) (end 39.8767 -42.9709) (width 0.3) (layer "F.Cu") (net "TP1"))
 (segment (start 38.525 -28.925) (end 37.1692 -30.2808) (width 0.3) (layer "F.Cu") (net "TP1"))
 (segment (start 37.1692 -30.2808) (end 37.1692 -40.2634) (width 0.3) (layer "F.Cu") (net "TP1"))
 (segment (start 39.8767 -88.7255) (end 36.0522 -92.55) (width 0.3) (layer "F.Cu") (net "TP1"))
 (segment (start 80.2587 -92.55) (end 51.8375 -64.1288) (width 0.3) (layer "F.Cu") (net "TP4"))
 (segment (start 51.8375 -64.1288) (end 51.8375 -38.2088) (width 0.3) (layer "F.Cu") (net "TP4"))
 (via (at 51.8375 -38.2088) (size 0.7) (drill 0.3) (layers "F.Cu" "B.Cu") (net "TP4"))
 (segment (start 51.8375 -38.2088) (end 47.5537 -33.925) (width 0.3) (layer "B.Cu") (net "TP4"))
 (segment (start 47.5537 -33.925) (end 38.525 -33.925) (width 0.3) (layer "B.Cu") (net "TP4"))
 (segment (start 36.6493 -53.625) (end 38.525 -53.625) (width 0.3) (layer "F.Cu") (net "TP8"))
 (segment (start 26.8243 -63.45) (end 36.6493 -53.625) (width 0.3) (layer "F.Cu") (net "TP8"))
 (segment (start 61.8324 -41.3324) (end 54.425 -33.925) (width 0.3) (layer "F.Cu") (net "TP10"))
 (segment (start 61.8324 -63.45) (end 61.8324 -41.3324) (width 0.3) (layer "F.Cu") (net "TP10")))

